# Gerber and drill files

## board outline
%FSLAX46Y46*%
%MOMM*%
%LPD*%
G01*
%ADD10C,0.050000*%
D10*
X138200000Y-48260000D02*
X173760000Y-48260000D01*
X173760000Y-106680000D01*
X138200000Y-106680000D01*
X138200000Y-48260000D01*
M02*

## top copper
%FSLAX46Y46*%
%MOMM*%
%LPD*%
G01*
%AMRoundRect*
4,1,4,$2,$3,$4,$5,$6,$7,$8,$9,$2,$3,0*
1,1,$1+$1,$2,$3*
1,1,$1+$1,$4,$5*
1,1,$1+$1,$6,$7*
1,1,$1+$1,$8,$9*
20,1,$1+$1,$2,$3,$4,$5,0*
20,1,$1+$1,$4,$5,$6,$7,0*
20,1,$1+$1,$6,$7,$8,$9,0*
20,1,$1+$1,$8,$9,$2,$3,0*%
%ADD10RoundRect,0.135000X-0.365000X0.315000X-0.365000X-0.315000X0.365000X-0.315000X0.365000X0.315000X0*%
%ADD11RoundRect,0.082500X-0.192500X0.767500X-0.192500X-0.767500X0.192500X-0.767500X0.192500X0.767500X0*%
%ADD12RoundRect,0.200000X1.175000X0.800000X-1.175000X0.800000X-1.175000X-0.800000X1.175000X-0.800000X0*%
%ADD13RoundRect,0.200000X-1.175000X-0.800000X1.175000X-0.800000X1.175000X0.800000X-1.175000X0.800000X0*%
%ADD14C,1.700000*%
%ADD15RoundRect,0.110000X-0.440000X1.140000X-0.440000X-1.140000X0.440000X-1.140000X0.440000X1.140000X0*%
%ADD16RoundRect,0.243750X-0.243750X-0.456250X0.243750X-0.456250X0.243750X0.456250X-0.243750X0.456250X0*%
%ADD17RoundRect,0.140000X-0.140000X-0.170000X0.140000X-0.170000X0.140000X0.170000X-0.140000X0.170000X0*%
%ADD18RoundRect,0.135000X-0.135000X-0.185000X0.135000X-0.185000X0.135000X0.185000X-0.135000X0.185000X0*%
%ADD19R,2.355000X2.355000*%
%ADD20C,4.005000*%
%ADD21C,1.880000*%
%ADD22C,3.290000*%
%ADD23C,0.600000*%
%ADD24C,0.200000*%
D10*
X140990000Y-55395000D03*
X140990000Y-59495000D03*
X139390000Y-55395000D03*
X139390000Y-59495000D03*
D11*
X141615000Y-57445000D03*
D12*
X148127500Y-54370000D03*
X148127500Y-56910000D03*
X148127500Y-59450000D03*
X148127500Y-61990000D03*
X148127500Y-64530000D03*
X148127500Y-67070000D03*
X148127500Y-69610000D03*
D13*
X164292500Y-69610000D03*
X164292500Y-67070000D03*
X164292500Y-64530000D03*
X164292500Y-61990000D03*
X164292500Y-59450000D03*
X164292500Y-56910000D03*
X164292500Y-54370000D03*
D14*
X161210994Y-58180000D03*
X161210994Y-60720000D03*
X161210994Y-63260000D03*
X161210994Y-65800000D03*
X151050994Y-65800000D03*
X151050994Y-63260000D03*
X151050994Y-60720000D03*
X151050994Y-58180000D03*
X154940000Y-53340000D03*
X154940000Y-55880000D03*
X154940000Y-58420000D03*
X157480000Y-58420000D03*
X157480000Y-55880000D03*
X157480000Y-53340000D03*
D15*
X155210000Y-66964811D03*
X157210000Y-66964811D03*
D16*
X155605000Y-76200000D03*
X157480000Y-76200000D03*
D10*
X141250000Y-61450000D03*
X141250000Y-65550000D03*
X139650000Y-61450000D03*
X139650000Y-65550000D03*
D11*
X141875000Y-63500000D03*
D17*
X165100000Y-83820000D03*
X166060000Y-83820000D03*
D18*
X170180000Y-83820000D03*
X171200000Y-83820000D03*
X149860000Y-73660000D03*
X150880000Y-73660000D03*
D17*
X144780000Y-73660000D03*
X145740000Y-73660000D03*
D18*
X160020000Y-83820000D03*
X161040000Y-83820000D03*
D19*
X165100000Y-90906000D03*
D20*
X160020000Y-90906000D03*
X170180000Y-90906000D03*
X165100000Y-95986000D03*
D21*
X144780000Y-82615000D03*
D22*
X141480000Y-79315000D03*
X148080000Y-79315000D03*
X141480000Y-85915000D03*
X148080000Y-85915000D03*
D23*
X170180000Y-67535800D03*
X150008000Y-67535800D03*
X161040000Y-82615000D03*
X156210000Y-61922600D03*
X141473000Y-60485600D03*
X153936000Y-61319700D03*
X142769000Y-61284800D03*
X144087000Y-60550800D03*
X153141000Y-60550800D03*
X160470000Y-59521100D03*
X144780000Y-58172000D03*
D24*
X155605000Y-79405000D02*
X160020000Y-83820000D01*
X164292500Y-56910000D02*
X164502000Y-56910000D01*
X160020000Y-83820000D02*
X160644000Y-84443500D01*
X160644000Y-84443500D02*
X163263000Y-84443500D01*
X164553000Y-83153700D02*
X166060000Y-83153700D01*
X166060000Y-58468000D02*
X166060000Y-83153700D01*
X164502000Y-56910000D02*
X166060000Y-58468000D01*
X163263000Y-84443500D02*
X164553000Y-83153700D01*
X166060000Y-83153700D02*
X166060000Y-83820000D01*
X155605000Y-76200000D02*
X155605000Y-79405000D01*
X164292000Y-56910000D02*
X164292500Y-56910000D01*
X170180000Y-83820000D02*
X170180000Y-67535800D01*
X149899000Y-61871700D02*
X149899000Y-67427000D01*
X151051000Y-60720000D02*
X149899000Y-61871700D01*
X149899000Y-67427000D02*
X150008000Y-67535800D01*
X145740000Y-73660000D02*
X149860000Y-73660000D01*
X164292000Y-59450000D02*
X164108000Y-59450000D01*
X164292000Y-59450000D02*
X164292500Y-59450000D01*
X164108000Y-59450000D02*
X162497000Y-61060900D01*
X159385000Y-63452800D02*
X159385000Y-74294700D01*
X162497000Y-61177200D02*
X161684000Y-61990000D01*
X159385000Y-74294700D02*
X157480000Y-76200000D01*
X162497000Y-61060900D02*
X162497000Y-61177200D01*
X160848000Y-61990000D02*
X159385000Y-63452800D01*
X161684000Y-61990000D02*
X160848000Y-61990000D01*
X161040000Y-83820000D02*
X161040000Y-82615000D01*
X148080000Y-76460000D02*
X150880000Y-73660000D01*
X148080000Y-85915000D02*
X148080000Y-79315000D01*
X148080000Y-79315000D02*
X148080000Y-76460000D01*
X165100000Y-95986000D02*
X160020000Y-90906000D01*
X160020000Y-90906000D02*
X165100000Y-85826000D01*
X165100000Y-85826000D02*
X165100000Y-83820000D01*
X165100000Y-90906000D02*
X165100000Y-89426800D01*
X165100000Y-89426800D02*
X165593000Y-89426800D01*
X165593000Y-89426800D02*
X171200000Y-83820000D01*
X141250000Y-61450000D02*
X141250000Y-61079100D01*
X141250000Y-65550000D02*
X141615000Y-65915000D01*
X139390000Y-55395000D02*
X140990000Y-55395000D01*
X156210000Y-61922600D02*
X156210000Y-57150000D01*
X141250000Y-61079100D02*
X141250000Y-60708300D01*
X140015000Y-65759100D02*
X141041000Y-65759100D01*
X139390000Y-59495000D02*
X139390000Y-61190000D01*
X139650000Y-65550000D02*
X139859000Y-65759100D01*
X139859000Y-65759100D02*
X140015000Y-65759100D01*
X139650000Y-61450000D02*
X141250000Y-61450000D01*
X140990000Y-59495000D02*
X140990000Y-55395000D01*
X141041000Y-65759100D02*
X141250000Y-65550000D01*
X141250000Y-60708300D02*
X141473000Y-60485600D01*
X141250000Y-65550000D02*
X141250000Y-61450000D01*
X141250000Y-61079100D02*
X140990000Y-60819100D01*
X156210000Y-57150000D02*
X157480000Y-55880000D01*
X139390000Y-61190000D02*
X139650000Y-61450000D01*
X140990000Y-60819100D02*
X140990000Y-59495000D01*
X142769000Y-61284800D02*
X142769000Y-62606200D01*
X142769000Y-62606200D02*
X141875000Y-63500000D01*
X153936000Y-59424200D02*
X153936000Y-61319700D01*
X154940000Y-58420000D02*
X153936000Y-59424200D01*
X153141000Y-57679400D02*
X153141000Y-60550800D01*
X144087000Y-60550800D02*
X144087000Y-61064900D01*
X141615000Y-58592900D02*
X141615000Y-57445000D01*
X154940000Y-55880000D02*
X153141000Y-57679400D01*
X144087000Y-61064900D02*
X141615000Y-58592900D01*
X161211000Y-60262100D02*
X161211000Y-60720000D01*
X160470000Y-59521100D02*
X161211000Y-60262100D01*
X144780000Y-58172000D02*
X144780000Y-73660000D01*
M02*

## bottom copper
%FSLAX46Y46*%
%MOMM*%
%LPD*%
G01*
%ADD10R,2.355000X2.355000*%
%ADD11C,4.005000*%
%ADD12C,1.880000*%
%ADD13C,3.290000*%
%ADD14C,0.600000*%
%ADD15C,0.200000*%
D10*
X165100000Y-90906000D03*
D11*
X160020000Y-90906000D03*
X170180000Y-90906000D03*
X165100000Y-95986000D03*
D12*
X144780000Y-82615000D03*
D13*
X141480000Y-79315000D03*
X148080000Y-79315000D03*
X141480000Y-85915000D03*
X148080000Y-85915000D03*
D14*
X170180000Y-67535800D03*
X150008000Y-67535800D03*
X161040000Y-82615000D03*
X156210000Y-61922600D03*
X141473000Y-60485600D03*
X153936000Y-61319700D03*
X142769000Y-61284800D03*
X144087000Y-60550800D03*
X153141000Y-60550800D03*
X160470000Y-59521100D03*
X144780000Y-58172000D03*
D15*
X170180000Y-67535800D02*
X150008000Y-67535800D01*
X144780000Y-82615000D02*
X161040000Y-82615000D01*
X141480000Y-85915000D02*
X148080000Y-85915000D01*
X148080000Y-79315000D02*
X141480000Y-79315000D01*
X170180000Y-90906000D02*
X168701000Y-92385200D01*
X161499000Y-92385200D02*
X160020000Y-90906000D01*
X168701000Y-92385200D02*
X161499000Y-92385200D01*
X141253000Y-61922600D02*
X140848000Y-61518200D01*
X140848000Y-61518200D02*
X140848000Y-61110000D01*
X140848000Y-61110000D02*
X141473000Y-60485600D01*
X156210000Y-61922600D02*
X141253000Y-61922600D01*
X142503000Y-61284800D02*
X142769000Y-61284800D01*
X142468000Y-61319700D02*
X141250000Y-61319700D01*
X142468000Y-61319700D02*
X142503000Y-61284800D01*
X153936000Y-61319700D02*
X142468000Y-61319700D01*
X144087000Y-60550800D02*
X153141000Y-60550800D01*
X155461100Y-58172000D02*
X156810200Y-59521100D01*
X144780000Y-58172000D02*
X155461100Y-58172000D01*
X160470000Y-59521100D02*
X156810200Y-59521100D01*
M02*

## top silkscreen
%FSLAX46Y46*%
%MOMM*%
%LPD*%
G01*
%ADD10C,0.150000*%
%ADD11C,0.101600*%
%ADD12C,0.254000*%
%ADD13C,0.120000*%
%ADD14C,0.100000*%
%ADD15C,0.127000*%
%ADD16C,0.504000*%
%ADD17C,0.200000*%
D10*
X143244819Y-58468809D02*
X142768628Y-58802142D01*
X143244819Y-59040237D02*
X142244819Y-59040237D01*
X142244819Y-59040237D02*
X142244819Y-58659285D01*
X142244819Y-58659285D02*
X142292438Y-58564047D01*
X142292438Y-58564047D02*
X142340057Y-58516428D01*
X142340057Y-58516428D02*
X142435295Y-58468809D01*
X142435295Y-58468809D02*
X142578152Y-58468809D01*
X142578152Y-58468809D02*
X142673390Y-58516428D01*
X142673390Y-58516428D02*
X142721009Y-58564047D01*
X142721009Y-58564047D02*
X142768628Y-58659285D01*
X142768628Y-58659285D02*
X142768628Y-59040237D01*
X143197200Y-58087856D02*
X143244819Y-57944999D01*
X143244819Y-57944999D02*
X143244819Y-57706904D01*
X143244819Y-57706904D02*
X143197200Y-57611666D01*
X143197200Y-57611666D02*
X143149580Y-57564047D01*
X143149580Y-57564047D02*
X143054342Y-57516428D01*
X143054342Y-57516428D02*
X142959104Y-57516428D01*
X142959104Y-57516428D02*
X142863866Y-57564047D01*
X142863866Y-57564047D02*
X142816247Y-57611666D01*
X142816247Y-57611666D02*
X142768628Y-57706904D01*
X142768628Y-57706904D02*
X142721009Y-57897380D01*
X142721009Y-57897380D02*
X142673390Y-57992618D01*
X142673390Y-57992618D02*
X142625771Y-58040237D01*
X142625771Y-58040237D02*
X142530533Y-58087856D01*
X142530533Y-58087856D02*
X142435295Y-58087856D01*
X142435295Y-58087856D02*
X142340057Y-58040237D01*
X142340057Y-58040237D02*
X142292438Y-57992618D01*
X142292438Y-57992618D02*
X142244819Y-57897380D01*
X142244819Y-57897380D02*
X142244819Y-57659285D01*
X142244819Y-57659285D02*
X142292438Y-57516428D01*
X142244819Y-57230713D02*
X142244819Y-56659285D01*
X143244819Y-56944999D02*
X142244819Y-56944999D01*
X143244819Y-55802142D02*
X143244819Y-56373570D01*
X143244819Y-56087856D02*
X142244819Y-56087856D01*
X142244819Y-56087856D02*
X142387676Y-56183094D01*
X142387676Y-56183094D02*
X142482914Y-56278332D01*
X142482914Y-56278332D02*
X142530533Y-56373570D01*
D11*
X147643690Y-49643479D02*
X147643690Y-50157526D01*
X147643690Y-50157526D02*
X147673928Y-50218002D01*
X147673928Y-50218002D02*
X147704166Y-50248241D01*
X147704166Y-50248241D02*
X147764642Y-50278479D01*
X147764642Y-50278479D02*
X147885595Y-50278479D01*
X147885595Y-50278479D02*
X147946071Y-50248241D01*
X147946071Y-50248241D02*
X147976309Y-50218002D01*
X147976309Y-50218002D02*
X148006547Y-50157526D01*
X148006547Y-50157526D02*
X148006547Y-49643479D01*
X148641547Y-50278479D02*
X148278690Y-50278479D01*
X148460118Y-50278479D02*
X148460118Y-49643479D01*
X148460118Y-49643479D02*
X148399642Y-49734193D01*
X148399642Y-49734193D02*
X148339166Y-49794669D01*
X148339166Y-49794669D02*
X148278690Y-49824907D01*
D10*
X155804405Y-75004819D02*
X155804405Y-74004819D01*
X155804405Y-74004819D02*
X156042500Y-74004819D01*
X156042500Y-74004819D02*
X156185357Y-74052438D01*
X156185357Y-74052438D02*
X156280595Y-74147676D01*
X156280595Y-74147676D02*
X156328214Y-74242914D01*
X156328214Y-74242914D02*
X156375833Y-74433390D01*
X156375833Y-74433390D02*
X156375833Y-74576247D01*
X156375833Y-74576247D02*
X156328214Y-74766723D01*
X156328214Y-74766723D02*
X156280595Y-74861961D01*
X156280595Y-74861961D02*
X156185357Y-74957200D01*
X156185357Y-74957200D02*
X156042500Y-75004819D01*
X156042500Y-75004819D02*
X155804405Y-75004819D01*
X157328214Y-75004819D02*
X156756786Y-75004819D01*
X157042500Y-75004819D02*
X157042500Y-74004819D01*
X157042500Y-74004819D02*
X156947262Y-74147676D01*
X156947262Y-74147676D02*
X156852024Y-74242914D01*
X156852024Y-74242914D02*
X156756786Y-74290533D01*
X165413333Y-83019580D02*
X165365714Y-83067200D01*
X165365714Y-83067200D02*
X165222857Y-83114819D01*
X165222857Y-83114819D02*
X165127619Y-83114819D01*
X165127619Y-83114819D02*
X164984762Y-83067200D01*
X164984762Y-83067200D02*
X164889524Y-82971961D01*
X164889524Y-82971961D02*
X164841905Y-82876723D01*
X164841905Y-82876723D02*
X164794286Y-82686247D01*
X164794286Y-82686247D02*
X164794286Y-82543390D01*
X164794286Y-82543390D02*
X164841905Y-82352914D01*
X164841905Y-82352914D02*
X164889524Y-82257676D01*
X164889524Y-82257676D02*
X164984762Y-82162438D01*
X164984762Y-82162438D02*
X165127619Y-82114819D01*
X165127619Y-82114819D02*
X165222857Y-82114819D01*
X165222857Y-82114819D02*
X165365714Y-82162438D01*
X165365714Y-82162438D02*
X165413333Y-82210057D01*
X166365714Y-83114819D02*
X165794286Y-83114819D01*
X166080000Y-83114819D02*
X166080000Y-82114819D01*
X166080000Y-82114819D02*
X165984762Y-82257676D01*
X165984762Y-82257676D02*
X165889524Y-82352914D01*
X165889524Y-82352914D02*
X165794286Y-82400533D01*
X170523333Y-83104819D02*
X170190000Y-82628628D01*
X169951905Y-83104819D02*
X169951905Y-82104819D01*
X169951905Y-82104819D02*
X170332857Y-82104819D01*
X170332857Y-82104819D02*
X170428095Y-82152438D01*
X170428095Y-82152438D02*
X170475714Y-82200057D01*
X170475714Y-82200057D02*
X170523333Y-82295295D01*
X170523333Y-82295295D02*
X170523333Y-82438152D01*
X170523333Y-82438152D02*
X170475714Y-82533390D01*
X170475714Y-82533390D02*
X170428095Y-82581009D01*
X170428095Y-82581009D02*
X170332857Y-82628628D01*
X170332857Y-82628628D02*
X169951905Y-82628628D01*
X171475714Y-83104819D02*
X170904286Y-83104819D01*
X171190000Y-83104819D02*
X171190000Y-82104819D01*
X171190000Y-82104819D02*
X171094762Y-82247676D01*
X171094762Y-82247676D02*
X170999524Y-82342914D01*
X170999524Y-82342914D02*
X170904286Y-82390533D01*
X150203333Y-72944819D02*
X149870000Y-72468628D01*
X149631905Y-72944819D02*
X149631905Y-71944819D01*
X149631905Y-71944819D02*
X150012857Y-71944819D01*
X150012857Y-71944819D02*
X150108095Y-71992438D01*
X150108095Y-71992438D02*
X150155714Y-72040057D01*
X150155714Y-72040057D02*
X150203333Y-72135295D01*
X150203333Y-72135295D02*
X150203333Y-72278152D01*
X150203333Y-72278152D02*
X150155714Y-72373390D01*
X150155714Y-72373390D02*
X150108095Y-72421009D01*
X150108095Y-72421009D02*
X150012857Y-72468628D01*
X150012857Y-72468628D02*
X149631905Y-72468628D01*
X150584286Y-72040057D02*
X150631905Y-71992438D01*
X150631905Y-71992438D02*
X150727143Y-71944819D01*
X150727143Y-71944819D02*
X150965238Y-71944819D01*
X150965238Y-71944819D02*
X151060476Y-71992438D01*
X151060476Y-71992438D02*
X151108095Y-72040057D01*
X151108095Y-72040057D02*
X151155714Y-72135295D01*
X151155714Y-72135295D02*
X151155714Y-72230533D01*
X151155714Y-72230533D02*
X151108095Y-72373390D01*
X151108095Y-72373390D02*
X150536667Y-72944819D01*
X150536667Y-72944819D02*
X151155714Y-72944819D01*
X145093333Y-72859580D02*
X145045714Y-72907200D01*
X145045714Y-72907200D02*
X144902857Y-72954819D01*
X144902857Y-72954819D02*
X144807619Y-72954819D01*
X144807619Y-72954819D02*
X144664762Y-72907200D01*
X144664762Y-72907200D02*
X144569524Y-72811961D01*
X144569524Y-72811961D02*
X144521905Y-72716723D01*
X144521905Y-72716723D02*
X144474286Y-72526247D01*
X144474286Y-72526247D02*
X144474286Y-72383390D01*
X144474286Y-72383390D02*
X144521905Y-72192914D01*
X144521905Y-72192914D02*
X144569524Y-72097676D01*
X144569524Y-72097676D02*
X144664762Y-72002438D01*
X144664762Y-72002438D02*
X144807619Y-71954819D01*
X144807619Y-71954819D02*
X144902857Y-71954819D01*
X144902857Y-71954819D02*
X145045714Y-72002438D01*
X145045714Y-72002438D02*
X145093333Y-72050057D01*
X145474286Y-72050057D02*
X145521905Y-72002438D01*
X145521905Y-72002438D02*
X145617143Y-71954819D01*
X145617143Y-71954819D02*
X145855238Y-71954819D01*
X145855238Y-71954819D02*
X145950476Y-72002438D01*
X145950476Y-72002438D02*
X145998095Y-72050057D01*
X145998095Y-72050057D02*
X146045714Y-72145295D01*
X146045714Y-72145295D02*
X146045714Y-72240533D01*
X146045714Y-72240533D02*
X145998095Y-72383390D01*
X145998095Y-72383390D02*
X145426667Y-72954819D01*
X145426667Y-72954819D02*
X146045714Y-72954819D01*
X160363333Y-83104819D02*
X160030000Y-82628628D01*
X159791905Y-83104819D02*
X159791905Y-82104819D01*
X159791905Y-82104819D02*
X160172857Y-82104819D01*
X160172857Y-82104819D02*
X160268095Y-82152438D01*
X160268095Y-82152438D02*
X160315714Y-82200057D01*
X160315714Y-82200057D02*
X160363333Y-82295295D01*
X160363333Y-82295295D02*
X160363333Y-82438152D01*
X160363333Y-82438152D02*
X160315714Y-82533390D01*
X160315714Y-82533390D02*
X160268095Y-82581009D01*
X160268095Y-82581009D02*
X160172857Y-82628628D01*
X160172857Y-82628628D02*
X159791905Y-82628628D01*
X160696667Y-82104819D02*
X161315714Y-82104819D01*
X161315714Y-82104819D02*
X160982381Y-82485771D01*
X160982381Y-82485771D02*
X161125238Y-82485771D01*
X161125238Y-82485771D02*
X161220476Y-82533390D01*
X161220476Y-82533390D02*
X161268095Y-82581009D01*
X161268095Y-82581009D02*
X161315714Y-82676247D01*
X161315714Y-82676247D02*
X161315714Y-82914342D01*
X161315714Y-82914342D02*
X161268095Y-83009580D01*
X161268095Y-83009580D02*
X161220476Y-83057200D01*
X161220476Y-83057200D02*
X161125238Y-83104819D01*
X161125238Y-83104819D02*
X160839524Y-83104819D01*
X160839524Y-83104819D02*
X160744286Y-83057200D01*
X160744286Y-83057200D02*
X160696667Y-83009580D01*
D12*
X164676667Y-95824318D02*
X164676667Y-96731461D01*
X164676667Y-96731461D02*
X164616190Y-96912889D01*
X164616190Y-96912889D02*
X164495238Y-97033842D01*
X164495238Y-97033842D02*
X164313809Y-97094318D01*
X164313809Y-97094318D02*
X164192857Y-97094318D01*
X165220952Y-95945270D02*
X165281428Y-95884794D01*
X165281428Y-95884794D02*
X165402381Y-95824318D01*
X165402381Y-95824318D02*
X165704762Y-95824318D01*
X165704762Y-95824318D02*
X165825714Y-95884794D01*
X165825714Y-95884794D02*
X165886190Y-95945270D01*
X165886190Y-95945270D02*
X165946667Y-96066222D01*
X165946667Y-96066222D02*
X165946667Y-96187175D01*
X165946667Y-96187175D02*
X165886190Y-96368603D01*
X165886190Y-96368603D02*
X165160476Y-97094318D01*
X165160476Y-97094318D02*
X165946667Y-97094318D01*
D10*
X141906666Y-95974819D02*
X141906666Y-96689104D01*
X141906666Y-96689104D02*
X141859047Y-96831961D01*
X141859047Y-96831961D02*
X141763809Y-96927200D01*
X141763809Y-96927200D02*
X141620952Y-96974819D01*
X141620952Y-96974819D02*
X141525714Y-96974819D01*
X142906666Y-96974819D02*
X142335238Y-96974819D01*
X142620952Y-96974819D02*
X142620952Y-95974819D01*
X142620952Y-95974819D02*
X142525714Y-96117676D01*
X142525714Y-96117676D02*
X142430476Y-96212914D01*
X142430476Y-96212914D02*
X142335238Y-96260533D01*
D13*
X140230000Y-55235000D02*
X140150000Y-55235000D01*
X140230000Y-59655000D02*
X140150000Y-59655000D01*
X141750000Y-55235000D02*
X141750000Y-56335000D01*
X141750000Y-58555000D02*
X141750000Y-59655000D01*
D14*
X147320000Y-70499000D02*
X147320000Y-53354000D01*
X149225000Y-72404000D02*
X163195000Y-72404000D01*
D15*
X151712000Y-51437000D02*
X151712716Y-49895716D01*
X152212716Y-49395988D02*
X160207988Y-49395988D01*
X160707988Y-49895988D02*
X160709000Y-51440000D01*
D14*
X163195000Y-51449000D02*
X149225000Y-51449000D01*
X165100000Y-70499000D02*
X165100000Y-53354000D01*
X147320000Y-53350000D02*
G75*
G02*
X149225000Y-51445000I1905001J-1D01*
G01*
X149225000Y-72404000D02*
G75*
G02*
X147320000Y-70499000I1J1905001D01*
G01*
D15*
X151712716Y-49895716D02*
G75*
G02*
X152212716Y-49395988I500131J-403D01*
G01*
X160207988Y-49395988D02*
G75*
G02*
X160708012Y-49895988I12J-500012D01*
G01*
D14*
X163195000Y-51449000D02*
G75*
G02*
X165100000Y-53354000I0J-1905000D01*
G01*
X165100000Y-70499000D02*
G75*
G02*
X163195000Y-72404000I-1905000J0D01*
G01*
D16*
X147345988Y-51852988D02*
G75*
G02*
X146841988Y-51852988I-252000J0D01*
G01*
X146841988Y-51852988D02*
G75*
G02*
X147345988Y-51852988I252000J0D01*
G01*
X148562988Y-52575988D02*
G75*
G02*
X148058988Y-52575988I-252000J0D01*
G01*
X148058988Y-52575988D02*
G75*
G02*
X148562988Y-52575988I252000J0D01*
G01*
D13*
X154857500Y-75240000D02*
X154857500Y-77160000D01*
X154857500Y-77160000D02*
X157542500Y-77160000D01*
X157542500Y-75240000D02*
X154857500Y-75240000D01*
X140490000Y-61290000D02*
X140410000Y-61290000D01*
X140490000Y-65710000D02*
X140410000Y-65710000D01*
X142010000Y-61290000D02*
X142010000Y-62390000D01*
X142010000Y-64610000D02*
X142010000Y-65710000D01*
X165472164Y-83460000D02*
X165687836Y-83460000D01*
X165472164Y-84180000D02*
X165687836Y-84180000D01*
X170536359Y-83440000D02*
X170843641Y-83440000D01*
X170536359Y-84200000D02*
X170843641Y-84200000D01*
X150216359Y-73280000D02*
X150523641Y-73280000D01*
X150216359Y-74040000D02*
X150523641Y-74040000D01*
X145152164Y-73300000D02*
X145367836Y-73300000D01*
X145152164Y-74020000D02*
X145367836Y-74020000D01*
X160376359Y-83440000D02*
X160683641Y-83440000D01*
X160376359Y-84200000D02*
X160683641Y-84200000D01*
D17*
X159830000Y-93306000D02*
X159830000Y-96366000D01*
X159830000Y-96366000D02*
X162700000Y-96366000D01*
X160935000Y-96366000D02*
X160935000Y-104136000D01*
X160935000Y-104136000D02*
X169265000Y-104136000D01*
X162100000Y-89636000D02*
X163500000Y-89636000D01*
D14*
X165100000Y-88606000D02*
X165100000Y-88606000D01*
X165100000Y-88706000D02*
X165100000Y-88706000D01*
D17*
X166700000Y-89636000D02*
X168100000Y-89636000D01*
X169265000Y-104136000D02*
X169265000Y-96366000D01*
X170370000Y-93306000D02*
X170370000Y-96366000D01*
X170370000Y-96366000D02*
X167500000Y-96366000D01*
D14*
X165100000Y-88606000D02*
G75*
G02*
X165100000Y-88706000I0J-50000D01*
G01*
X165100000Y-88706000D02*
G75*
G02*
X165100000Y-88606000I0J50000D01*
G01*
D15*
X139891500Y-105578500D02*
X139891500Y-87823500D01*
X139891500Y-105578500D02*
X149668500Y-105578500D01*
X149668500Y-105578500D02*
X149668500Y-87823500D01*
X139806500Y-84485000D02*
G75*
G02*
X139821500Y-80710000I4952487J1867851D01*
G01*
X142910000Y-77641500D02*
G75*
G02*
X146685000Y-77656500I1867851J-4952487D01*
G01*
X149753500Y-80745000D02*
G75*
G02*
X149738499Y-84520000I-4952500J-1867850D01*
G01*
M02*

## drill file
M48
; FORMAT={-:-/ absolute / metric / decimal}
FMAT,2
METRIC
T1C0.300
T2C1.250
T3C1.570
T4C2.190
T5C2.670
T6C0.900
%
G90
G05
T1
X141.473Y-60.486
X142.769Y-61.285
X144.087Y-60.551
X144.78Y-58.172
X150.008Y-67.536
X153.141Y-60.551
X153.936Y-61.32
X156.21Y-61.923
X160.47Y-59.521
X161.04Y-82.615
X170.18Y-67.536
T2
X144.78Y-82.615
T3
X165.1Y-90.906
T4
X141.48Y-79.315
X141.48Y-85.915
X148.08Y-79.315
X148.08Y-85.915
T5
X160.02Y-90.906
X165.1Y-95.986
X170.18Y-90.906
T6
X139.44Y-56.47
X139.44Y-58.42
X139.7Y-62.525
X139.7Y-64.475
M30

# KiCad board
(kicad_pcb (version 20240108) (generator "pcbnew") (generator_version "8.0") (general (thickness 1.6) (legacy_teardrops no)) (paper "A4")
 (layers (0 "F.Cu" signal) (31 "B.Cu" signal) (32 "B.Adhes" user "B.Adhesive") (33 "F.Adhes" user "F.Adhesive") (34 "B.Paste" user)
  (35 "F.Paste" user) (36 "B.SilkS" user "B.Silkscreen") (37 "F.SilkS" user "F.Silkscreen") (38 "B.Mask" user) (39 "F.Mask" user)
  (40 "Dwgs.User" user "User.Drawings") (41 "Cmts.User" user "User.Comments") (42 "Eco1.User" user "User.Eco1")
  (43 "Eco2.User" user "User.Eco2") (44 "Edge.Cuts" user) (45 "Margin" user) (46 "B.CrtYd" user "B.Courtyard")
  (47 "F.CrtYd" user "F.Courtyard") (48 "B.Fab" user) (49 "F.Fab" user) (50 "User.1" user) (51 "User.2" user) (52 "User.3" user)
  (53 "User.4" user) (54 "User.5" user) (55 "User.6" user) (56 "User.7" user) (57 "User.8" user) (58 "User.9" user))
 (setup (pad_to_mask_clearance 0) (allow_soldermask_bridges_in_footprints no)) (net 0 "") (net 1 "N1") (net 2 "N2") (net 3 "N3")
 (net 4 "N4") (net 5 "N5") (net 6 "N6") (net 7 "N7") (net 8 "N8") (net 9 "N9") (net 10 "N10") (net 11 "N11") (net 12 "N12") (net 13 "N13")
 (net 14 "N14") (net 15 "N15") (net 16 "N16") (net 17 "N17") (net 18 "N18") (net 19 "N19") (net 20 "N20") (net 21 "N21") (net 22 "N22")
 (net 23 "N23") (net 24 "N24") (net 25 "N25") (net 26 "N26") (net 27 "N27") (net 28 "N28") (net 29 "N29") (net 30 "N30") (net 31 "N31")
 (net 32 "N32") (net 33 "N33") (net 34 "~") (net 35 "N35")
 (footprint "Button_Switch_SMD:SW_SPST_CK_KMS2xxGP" (layer "F.Cu") (at 140.19 57.445 -90)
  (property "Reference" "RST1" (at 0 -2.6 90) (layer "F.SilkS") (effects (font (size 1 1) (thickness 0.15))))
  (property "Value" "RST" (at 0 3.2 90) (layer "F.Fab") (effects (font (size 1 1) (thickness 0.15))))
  (fp_line (start -2.21 -0.04) (end -2.21 0.04) (stroke (width 0.12) (type default)) (layer "F.SilkS"))
  (fp_line (start 2.21 -0.04) (end 2.21 0.04) (stroke (width 0.12) (type default)) (layer "F.SilkS"))
  (fp_line (start -2.21 -1.56) (end -1.11 -1.56) (stroke (width 0.12) (type solid)) (layer "F.SilkS"))
  (fp_line (start 1.11 -1.56) (end 2.21 -1.56) (stroke (width 0.12) (type solid)) (layer "F.SilkS"))
  (pad "" np_thru_hole circle (at -0.975 0.75 270) (size 0.9 0.9) (drill 0.9) (layers "F&B.Cu" "*.Mask"))
  (pad "" np_thru_hole circle (at 0.975 0.75 270) (size 0.9 0.9) (drill 0.9) (layers "F&B.Cu" "*.Mask"))
  (pad "1" smd roundrect (at -2.05 -0.8 270) (size 0.9 1) (layers "F.Cu" "F.Paste" "F.Mask") (roundrect_rratio 0.15) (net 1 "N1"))
  (pad "1" smd roundrect (at 2.05 -0.8 270) (size 0.9 1) (layers "F.Cu" "F.Paste" "F.Mask") (roundrect_rratio 0.15) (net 1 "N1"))
  (pad "2" smd roundrect (at -2.05 0.8 270) (size 0.9 1) (layers "F.Cu" "F.Paste" "F.Mask") (roundrect_rratio 0.15) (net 1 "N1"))
  (pad "2" smd roundrect (at 2.05 0.8 270) (size 0.9 1) (layers "F.Cu" "F.Paste" "F.Mask") (roundrect_rratio 0.15) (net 1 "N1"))
  (pad "SH" smd roundrect (at 0 -1.425 270) (size 1.7 0.55) (layers "F.Cu" "F.Paste" "F.Mask") (roundrect_rratio 0.15) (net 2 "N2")))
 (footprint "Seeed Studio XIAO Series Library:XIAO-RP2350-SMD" (layer "F.Cu") (at 156.1275 61.99)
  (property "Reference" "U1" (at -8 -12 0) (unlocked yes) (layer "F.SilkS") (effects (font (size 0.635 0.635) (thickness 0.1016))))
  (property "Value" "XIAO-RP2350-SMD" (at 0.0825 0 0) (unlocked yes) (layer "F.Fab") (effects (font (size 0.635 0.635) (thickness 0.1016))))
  (fp_line (start -8.8075 8.509) (end -8.8075 -8.636) (stroke (width 0.1) (type solid)) (layer "F.SilkS"))
  (fp_line (start -6.9025 10.414) (end 7.0675 10.414) (stroke (width 0.1) (type solid)) (layer "F.SilkS"))
  (fp_line (start -4.4155 -10.553) (end -4.414784 -12.094284) (stroke (width 0.127) (type solid)) (layer "F.SilkS"))
  (fp_line (start -3.914784 -12.594012) (end 4.080488 -12.594012) (stroke (width 0.127) (type solid)) (layer "F.SilkS"))
  (fp_line (start 4.580488 -12.094012) (end 4.5815 -10.55) (stroke (width 0.127) (type solid)) (layer "F.SilkS"))
  (fp_line (start 7.0675 -10.541) (end -6.9025 -10.541) (stroke (width 0.1) (type solid)) (layer "F.SilkS"))
  (fp_line (start 8.9725 8.509) (end 8.9725 -8.636) (stroke (width 0.1) (type solid)) (layer "F.SilkS"))
  (fp_arc (start -8.8075 -8.64) (mid -8.249538 -9.987038) (end -6.9025 -10.545) (stroke (width 0.1) (type solid)) (layer "F.SilkS"))
  (fp_arc (start -6.9025 10.414) (mid -8.249538 9.856038) (end -8.8075 8.509) (stroke (width 0.1) (type solid)) (layer "F.SilkS"))
  (fp_arc (start -4.414784 -12.094284) (mid -4.268203 -12.447623) (end -3.914784 -12.594012) (stroke (width 0.127) (type default))
   (layer "F.SilkS"))
  (fp_arc (start 4.080488 -12.594012) (mid 4.434053 -12.44757) (end 4.580488 -12.094012) (stroke (width 0.127) (type default))
   (layer "F.SilkS"))
  (fp_arc (start 7.0675 -10.541) (mid 8.414538 -9.983038) (end 8.9725 -8.636) (stroke (width 0.1) (type solid)) (layer "F.SilkS"))
  (fp_arc (start 8.9725 8.509) (mid 8.414538 9.856038) (end 7.0675 10.414) (stroke (width 0.1) (type solid)) (layer "F.SilkS"))
  (fp_circle (center -9.033512 -10.137012) (end -9.033512 -10.391012) (stroke (width 0.5) (type solid)) (fill solid) (layer "F.SilkS"))
  (fp_circle (center -7.816512 -9.414012) (end -7.816512 -9.668012) (stroke (width 0.5) (type solid)) (fill solid) (layer "F.SilkS"))
  (pad "1" smd roundrect (at -8 -7.62 180) (size 2.75 2) (layers "F.Cu" "F.Paste" "F.Mask") (roundrect_rratio 0.1) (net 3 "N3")
   (thermal_bridge_angle 45))
  (pad "2" smd roundrect (at -8 -5.08 180) (size 2.75 2) (layers "F.Cu" "F.Paste" "F.Mask") (roundrect_rratio 0.1) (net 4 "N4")
   (thermal_bridge_angle 45))
  (pad "3" smd roundrect (at -8 -2.54 180) (size 2.75 2) (layers "F.Cu" "F.Paste" "F.Mask") (roundrect_rratio 0.1) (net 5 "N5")
   (thermal_bridge_angle 45))
  (pad "4" smd roundrect (at -8 0 180) (size 2.75 2) (layers "F.Cu" "F.Paste" "F.Mask") (roundrect_rratio 0.1) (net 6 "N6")
   (thermal_bridge_angle 45))
  (pad "5" smd roundrect (at -8 2.54 180) (size 2.75 2) (layers "F.Cu" "F.Paste" "F.Mask") (roundrect_rratio 0.1) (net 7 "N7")
   (thermal_bridge_angle 45))
  (pad "6" smd roundrect (at -8 5.08 180) (size 2.75 2) (layers "F.Cu" "F.Paste" "F.Mask") (roundrect_rratio 0.1) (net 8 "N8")
   (thermal_bridge_angle 45))
  (pad "7" smd roundrect (at -8 7.62 180) (size 2.75 2) (layers "F.Cu" "F.Paste" "F.Mask") (roundrect_rratio 0.1) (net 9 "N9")
   (thermal_bridge_angle 45))
  (pad "8" smd roundrect (at 8.165 7.62) (size 2.75 2) (layers "F.Cu" "F.Paste" "F.Mask") (roundrect_rratio 0.1) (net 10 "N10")
   (thermal_bridge_angle 45))
  (pad "9" smd roundrect (at 8.165 5.08) (size 2.75 2) (layers "F.Cu" "F.Paste" "F.Mask") (roundrect_rratio 0.1) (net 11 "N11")
   (thermal_bridge_angle 45))
  (pad "10" smd roundrect (at 8.165 2.54) (size 2.75 2) (layers "F.Cu" "F.Paste" "F.Mask") (roundrect_rratio 0.1) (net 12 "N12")
   (thermal_bridge_angle 45))
  (pad "11" smd roundrect (at 8.165 0) (size 2.75 2) (layers "F.Cu" "F.Paste" "F.Mask") (roundrect_rratio 0.1) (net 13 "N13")
   (thermal_bridge_angle 45))
  (pad "12" smd roundrect (at 8.165 -2.54) (size 2.75 2) (layers "F.Cu" "F.Paste" "F.Mask") (roundrect_rratio 0.1) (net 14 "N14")
   (thermal_bridge_angle 45))
  (pad "13" smd roundrect (at 8.165 -5.08) (size 2.75 2) (layers "F.Cu" "F.Paste" "F.Mask") (roundrect_rratio 0.1) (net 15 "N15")
   (thermal_bridge_angle 45))
  (pad "14" smd roundrect (at 8.165 -7.62) (size 2.75 2) (layers "F.Cu" "F.Paste" "F.Mask") (roundrect_rratio 0.1) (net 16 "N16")
   (thermal_bridge_angle 45))
  (pad "15" smd circle (at 5.083494 -3.81 180) (size 1.7 1.7) (layers "F.Cu" "F.Paste" "F.Mask") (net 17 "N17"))
  (pad "16" smd circle (at 5.083494 -1.27 180) (size 1.7 1.7) (layers "F.Cu" "F.Paste" "F.Mask") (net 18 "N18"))
  (pad "17" smd circle (at 5.083494 1.27 180) (size 1.7 1.7) (layers "F.Cu" "F.Paste" "F.Mask") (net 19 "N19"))
  (pad "18" smd circle (at 5.083494 3.81 180) (size 1.7 1.7) (layers "F.Cu" "F.Paste" "F.Mask") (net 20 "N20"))
  (pad "19" smd circle (at -5.076506 3.81 180) (size 1.7 1.7) (layers "F.Cu" "F.Paste" "F.Mask") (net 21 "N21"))
  (pad "20" smd circle (at -5.076506 1.27 180) (size 1.7 1.7) (layers "F.Cu" "F.Paste" "F.Mask") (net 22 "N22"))
  (pad "21" smd circle (at -5.076506 -1.27 180) (size 1.7 1.7) (layers "F.Cu" "F.Paste" "F.Mask") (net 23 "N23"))
  (pad "22" smd circle (at -5.076506 -3.81 180) (size 1.7 1.7) (layers "F.Cu" "F.Paste" "F.Mask") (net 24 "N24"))
  (pad "23" smd circle (at -1.1875 -8.65 180) (size 1.7 1.7) (layers "F.Cu" "F.Paste" "F.Mask") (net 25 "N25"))
  (pad "24" smd circle (at -1.1875 -6.11 180) (size 1.7 1.7) (layers "F.Cu" "F.Paste" "F.Mask") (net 2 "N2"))
  (pad "25" smd circle (at -1.1875 -3.57 180) (size 1.7 1.7) (layers "F.Cu" "F.Paste" "F.Mask") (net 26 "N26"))
  (pad "26" smd circle (at 1.3525 -3.57 180) (size 1.7 1.7) (layers "F.Cu" "F.Paste" "F.Mask") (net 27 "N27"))
  (pad "27" smd circle (at 1.3525 -6.11 180) (size 1.7 1.7) (layers "F.Cu" "F.Paste" "F.Mask") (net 1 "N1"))
  (pad "28" smd circle (at 1.3525 -8.65 180) (size 1.7 1.7) (layers "F.Cu" "F.Paste" "F.Mask") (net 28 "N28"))
  (pad "29" smd roundrect (at -0.9175 4.974811 270) (size 2.5 1.1) (layers "F.Cu" "F.Paste" "F.Mask") (roundrect_rratio 0.1) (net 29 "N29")
   (thermal_bridge_angle 45))
  (pad "30" smd roundrect (at 1.0825 4.974811 270) (size 2.5 1.1) (layers "F.Cu" "F.Paste" "F.Mask") (roundrect_rratio 0.1) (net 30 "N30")
   (thermal_bridge_angle 45)))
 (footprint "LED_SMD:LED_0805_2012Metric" (layer "F.Cu") (at 156.5425 76.2)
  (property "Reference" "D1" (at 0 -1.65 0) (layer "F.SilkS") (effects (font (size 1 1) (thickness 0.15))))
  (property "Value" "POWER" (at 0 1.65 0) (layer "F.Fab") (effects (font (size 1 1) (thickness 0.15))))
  (fp_line (start -1.685 -0.96) (end -1.685 0.96) (stroke (width 0.12) (type solid)) (layer "F.SilkS"))
  (fp_line (start -1.685 0.96) (end 1 0.96) (stroke (width 0.12) (type solid)) (layer "F.SilkS"))
  (fp_line (start 1 -0.96) (end -1.685 -0.96) (stroke (width 0.12) (type solid)) (layer "F.SilkS"))
  (pad "1" smd roundrect (at -0.9375 0) (size 0.975 1.4) (layers "F.Cu" "F.Paste" "F.Mask") (roundrect_rratio 0.25) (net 15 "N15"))
  (pad "2" smd roundrect (at 0.9375 0) (size 0.975 1.4) (layers "F.Cu" "F.Paste" "F.Mask") (roundrect_rratio 0.25) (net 14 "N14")))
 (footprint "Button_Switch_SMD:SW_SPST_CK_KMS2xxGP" (layer "F.Cu") (at 140.45 63.5 -90)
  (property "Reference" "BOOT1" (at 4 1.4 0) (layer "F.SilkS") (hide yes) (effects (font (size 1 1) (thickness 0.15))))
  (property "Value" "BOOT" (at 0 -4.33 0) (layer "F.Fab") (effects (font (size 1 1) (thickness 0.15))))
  (fp_line (start -2.21 -0.04) (end -2.21 0.04) (stroke (width 0.12) (type default)) (layer "F.SilkS"))
  (fp_line (start 2.21 -0.04) (end 2.21 0.04) (stroke (width 0.12) (type default)) (layer "F.SilkS"))
  (fp_line (start -2.21 -1.56) (end -1.11 -1.56) (stroke (width 0.12) (type solid)) (layer "F.SilkS"))
  (fp_line (start 1.11 -1.56) (end 2.21 -1.56) (stroke (width 0.12) (type solid)) (layer "F.SilkS"))
  (pad "" np_thru_hole circle (at -0.975 0.75 270) (size 0.9 0.9) (drill 0.9) (layers "F&B.Cu" "*.Mask"))
  (pad "" np_thru_hole circle (at 0.975 0.75 270) (size 0.9 0.9) (drill 0.9) (layers "F&B.Cu" "*.Mask"))
  (pad "1" smd roundrect (at -2.05 -0.8 270) (size 0.9 1) (layers "F.Cu" "F.Paste" "F.Mask") (roundrect_rratio 0.15) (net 1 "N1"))
  (pad "1" smd roundrect (at 2.05 -0.8 270) (size 0.9 1) (layers "F.Cu" "F.Paste" "F.Mask") (roundrect_rratio 0.15) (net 1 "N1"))
  (pad "2" smd roundrect (at -2.05 0.8 270) (size 0.9 1) (layers "F.Cu" "F.Paste" "F.Mask") (roundrect_rratio 0.15) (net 1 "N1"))
  (pad "2" smd roundrect (at 2.05 0.8 270) (size 0.9 1) (layers "F.Cu" "F.Paste" "F.Mask") (roundrect_rratio 0.15) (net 1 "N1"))
  (pad "SH" smd roundrect (at 0 -1.425 270) (size 1.7 0.55) (layers "F.Cu" "F.Paste" "F.Mask") (roundrect_rratio 0.15) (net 26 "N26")))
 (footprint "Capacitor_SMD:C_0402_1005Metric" (layer "F.Cu") (at 165.58 83.82)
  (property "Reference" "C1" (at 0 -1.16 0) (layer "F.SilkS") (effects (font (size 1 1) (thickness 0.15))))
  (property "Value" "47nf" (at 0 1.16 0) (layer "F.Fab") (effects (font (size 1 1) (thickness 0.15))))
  (fp_line (start -0.107836 -0.36) (end 0.107836 -0.36) (stroke (width 0.12) (type solid)) (layer "F.SilkS"))
  (fp_line (start -0.107836 0.36) (end 0.107836 0.36) (stroke (width 0.12) (type solid)) (layer "F.SilkS"))
  (pad "1" smd roundrect (at -0.48 0) (size 0.56 0.62) (layers "F.Cu" "F.Paste" "F.Mask") (roundrect_rratio 0.25) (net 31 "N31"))
  (pad "2" smd roundrect (at 0.48 0) (size 0.56 0.62) (layers "F.Cu" "F.Paste" "F.Mask") (roundrect_rratio 0.25) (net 15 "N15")))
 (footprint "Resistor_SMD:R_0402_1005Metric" (layer "F.Cu") (at 170.69 83.82)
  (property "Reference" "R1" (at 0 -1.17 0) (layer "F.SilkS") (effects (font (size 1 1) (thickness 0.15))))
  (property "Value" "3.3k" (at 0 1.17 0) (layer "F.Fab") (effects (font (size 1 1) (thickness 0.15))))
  (fp_line (start -0.153641 -0.38) (end 0.153641 -0.38) (stroke (width 0.12) (type solid)) (layer "F.SilkS"))
  (fp_line (start -0.153641 0.38) (end 0.153641 0.38) (stroke (width 0.12) (type solid)) (layer "F.SilkS"))
  (pad "1" smd roundrect (at -0.51 0) (size 0.54 0.64) (layers "F.Cu" "F.Paste" "F.Mask") (roundrect_rratio 0.25) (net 23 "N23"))
  (pad "2" smd roundrect (at 0.51 0) (size 0.54 0.64) (layers "F.Cu" "F.Paste" "F.Mask") (roundrect_rratio 0.25) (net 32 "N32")))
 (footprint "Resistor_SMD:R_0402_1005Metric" (layer "F.Cu") (at 150.37 73.66)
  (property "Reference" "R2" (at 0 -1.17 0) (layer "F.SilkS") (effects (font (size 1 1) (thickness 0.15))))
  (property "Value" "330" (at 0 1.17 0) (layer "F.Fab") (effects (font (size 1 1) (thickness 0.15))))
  (fp_line (start -0.153641 -0.38) (end 0.153641 -0.38) (stroke (width 0.12) (type solid)) (layer "F.SilkS"))
  (fp_line (start -0.153641 0.38) (end 0.153641 0.38) (stroke (width 0.12) (type solid)) (layer "F.SilkS"))
  (pad "1" smd roundrect (at -0.51 0) (size 0.54 0.64) (layers "F.Cu" "F.Paste" "F.Mask") (roundrect_rratio 0.25) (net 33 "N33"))
  (pad "2" smd roundrect (at 0.51 0) (size 0.54 0.64) (layers "F.Cu" "F.Paste" "F.Mask") (roundrect_rratio 0.25) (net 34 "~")))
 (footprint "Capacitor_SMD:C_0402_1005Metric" (layer "F.Cu") (at 145.26 73.66)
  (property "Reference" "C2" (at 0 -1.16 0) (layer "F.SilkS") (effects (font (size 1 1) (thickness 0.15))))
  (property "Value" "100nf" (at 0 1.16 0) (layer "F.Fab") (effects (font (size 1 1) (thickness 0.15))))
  (fp_line (start -0.107836 -0.36) (end 0.107836 -0.36) (stroke (width 0.12) (type solid)) (layer "F.SilkS"))
  (fp_line (start -0.107836 0.36) (end 0.107836 0.36) (stroke (width 0.12) (type solid)) (layer "F.SilkS"))
  (pad "1" smd roundrect (at -0.48 0) (size 0.56 0.62) (layers "F.Cu" "F.Paste" "F.Mask") (roundrect_rratio 0.25) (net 18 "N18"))
  (pad "2" smd roundrect (at 0.48 0) (size 0.56 0.62) (layers "F.Cu" "F.Paste" "F.Mask") (roundrect_rratio 0.25) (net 33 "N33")))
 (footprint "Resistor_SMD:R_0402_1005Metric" (layer "F.Cu") (at 160.53 83.82)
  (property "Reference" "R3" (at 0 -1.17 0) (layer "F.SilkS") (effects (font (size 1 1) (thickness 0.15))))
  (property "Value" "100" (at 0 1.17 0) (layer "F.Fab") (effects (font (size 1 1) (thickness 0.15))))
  (fp_line (start -0.153641 -0.38) (end 0.153641 -0.38) (stroke (width 0.12) (type solid)) (layer "F.SilkS"))
  (fp_line (start -0.153641 0.38) (end 0.153641 0.38) (stroke (width 0.12) (type solid)) (layer "F.SilkS"))
  (pad "1" smd roundrect (at -0.51 0) (size 0.54 0.64) (layers "F.Cu" "F.Paste" "F.Mask") (roundrect_rratio 0.25) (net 15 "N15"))
  (pad "2" smd roundrect (at 0.51 0) (size 0.54 0.64) (layers "F.Cu" "F.Paste" "F.Mask") (roundrect_rratio 0.25) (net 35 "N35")))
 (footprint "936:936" (layer "F.Cu") (at 165.1 90.906)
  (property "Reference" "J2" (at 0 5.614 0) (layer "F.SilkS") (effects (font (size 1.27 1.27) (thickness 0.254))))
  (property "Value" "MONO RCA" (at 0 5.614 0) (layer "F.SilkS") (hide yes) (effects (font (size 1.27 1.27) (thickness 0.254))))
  (fp_line (start -5.27 2.4) (end -5.27 5.46) (stroke (width 0.2) (type solid)) (layer "F.SilkS"))
  (fp_line (start -5.27 5.46) (end -2.4 5.46) (stroke (width 0.2) (type solid)) (layer "F.SilkS"))
  (fp_line (start -4.165 5.46) (end -4.165 13.23) (stroke (width 0.2) (type solid)) (layer "F.SilkS"))
  (fp_line (start -4.165 13.23) (end 4.165 13.23) (stroke (width 0.2) (type solid)) (layer "F.SilkS"))
  (fp_line (start -3 -1.27) (end -1.6 -1.27) (stroke (width 0.2) (type solid)) (layer "F.SilkS"))
  (fp_line (start 0 -2.3) (end 0 -2.3) (stroke (width 0.1) (type solid)) (layer "F.SilkS"))
  (fp_line (start 0 -2.2) (end 0 -2.2) (stroke (width 0.1) (type solid)) (layer "F.SilkS"))
  (fp_line (start 1.6 -1.27) (end 3 -1.27) (stroke (width 0.2) (type solid)) (layer "F.SilkS"))
  (fp_line (start 4.165 13.23) (end 4.165 5.46) (stroke (width 0.2) (type solid)) (layer "F.SilkS"))
  (fp_line (start 5.27 2.4) (end 5.27 5.46) (stroke (width 0.2) (type solid)) (layer "F.SilkS"))
  (fp_line (start 5.27 5.46) (end 2.4 5.46) (stroke (width 0.2) (type solid)) (layer "F.SilkS"))
  (fp_arc (start 0 -2.3) (mid 0.05 -2.25) (end 0 -2.2) (stroke (width 0.1) (type solid)) (layer "F.SilkS"))
  (fp_arc (start 0 -2.2) (mid -0.05 -2.25) (end 0 -2.3) (stroke (width 0.1) (type solid)) (layer "F.SilkS"))
  (pad "1" thru_hole rect (at 0 0) (size 2.355 2.355) (drill 1.57) (layers "*.Cu" "*.Mask") (remove_unused_layers no) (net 32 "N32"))
  (pad "MH1" thru_hole circle (at -5.08 0) (size 4.005 4.005) (drill 2.67) (layers "*.Cu" "*.Mask") (remove_unused_layers no) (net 31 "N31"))
  (pad "MH2" thru_hole circle (at 5.08 0) (size 4.005 4.005) (drill 2.67) (layers "*.Cu" "*.Mask") (remove_unused_layers no) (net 31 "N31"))
  (pad "MH3" thru_hole circle (at 0 5.08) (size 4.005 4.005) (drill 2.67) (layers "*.Cu" "*.Mask") (remove_unused_layers no) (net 31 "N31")))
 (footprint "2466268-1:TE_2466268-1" (layer "F.Cu") (at 144.78 82.615)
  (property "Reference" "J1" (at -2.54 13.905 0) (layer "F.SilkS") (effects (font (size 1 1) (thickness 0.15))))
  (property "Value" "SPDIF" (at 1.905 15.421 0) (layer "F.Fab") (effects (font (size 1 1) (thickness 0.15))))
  (fp_line (start -4.8885 22.9635) (end -4.8885 5.2085) (stroke (width 0.127) (type solid)) (layer "F.SilkS"))
  (fp_line (start -4.8885 22.9635) (end 4.8885 22.9635) (stroke (width 0.127) (type solid)) (layer "F.SilkS"))
  (fp_line (start 4.8885 22.9635) (end 4.8885 5.2085) (stroke (width 0.127) (type solid)) (layer "F.SilkS"))
  (fp_arc (start -4.9735 1.87) (mid -5.313985 -0.018883) (end -4.9585 -1.905) (stroke (width 0.127) (type solid)) (layer "F.SilkS"))
  (fp_arc (start -1.87 -4.9735) (mid 0.018883 -5.313985) (end 1.905 -4.9585) (stroke (width 0.127) (type solid)) (layer "F.SilkS"))
  (fp_arc (start 4.9735 -1.87) (mid 5.313984 0.018883) (end 4.9585 1.905) (stroke (width 0.127) (type solid)) (layer "F.SilkS"))
  (pad "1" thru_hole circle (at 0 0) (size 1.88 1.88) (drill 1.25) (layers "*.Cu" "*.Mask") (remove_unused_layers no) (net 35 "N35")
   (solder_mask_margin 0.102))
  (pad "2" thru_hole circle (at -3.3 -3.3) (size 3.29 3.29) (drill 2.19) (layers "*.Cu" "*.Mask") (remove_unused_layers no) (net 34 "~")
   (solder_mask_margin 0.102))
  (pad "3" thru_hole circle (at 3.3 -3.3) (size 3.29 3.29) (drill 2.19) (layers "*.Cu" "*.Mask") (remove_unused_layers no) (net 34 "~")
   (solder_mask_margin 0.102))
  (pad "4" thru_hole circle (at -3.3 3.3) (size 3.29 3.29) (drill 2.19) (layers "*.Cu" "*.Mask") (remove_unused_layers no) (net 34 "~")
   (solder_mask_margin 0.102))
  (pad "5" thru_hole circle (at 3.3 3.3) (size 3.29 3.29) (drill 2.19) (layers "*.Cu" "*.Mask") (remove_unused_layers no) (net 34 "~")
   (solder_mask_margin 0.102)))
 (gr_rect (start 138.2 48.26) (end 173.76 106.68) (stroke (width 0.05) (type default)) (fill none) (layer "Edge.Cuts"))
 (segment (start 155.605 79.405) (end 160.02 83.82) (width 0.2) (layer "F.Cu") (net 15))
 (segment (start 164.2925 56.91) (end 164.502 56.91) (width 0.2) (layer "F.Cu") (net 15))
 (segment (start 160.02 83.82) (end 160.644 84.4435) (width 0.2) (layer "F.Cu") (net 15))
 (segment (start 160.644 84.4435) (end 163.263 84.4435) (width 0.2) (layer "F.Cu") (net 15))
 (segment (start 164.553 83.1537) (end 166.06 83.1537) (width 0.2) (layer "F.Cu") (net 15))
 (segment (start 166.06 58.468) (end 166.06 83.1537) (width 0.2) (layer "F.Cu") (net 15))
 (segment (start 164.502 56.91) (end 166.06 58.468) (width 0.2) (layer "F.Cu") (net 15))
 (segment (start 163.263 84.4435) (end 164.553 83.1537) (width 0.2) (layer "F.Cu") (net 15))
 (segment (start 166.06 83.1537) (end 166.06 83.82) (width 0.2) (layer "F.Cu") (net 15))
 (segment (start 155.605 76.2) (end 155.605 79.405) (width 0.2) (layer "F.Cu") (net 15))
 (segment (start 164.292 56.91) (end 164.2925 56.91) (width 0.2) (layer "F.Cu") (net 15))
 (segment (start 170.18 83.82) (end 170.18 67.5358) (width 0.2) (layer "F.Cu") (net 23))
 (segment (start 149.899 61.8717) (end 149.899 67.427) (width 0.2) (layer "F.Cu") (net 23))
 (segment (start 151.051 60.72) (end 149.899 61.8717) (width 0.2) (layer "F.Cu") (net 23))
 (segment (start 149.899 67.427) (end 150.008 67.5358) (width 0.2) (layer "F.Cu") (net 23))
 (via (at 170.18 67.5358) (size 0.6) (drill 0.3) (layers "F.Cu" "B.Cu") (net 23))
 (via (at 150.008 67.5358) (size 0.6) (drill 0.3) (layers "F.Cu" "B.Cu") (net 23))
 (segment (start 170.18 67.5358) (end 150.008 67.5358) (width 0.2) (layer "B.Cu") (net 23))
 (segment (start 145.74 73.66) (end 149.86 73.66) (width 0.2) (layer "F.Cu") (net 33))
 (segment (start 164.292 59.45) (end 164.108 59.45) (width 0.2) (layer "F.Cu") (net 14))
 (segment (start 164.292 59.45) (end 164.2925 59.45) (width 0.2) (layer "F.Cu") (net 14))
 (segment (start 164.108 59.45) (end 162.497 61.0609) (width 0.2) (layer "F.Cu") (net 14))
 (segment (start 159.385 63.4528) (end 159.385 74.2947) (width 0.2) (layer "F.Cu") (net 14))
 (segment (start 162.497 61.1772) (end 161.684 61.99) (width 0.2) (layer "F.Cu") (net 14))
 (segment (start 159.385 74.2947) (end 157.48 76.2) (width 0.2) (layer "F.Cu") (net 14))
 (segment (start 162.497 61.0609) (end 162.497 61.1772) (width 0.2) (layer "F.Cu") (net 14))
 (segment (start 160.848 61.99) (end 159.385 63.4528) (width 0.2) (layer "F.Cu") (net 14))
 (segment (start 161.684 61.99) (end 160.848 61.99) (width 0.2) (layer "F.Cu") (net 14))
 (segment (start 161.04 83.82) (end 161.04 82.615) (width 0.2) (layer "F.Cu") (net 35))
 (via (at 161.04 82.615) (size 0.6) (drill 0.3) (layers "F.Cu" "B.Cu") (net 35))
 (segment (start 144.78 82.615) (end 161.04 82.615) (width 0.2) (layer "B.Cu") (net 35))
 (segment (start 148.08 76.46) (end 150.88 73.66) (width 0.2) (layer "F.Cu") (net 34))
 (segment (start 148.08 85.915) (end 148.08 79.315) (width 0.2) (layer "F.Cu") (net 34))
 (segment (start 148.08 79.315) (end 148.08 76.46) (width 0.2) (layer "F.Cu") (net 34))
 (segment (start 141.48 85.915) (end 148.08 85.915) (width 0.2) (layer "B.Cu") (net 34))
 (segment (start 148.08 79.315) (end 141.48 79.315) (width 0.2) (layer "B.Cu") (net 34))
 (segment (start 165.1 95.986) (end 160.02 90.906) (width 0.2) (layer "F.Cu") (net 31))
 (segment (start 160.02 90.906) (end 165.1 85.826) (width 0.2) (layer "F.Cu") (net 31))
 (segment (start 165.1 85.826) (end 165.1 83.82) (width 0.2) (layer "F.Cu") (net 31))
 (segment (start 170.18 90.906) (end 168.701 92.3852) (width 0.2) (layer "B.Cu") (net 31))
 (segment (start 161.499 92.3852) (end 160.02 90.906) (width 0.2) (layer "B.Cu") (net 31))
 (segment (start 168.701 92.3852) (end 161.499 92.3852) (width 0.2) (layer "B.Cu") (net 31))
 (segment (start 165.1 90.906) (end 165.1 89.4268) (width 0.2) (layer "F.Cu") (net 32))
 (segment (start 165.1 89.4268) (end 165.593 89.4268) (width 0.2) (layer "F.Cu") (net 32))
 (segment (start 165.593 89.4268) (end 171.2 83.82) (width 0.2) (layer "F.Cu") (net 32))
 (segment (start 141.25 61.45) (end 141.25 61.0791) (width 0.2) (layer "F.Cu") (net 1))
 (segment (start 141.25 65.55) (end 141.615 65.915) (width 0.2) (layer "F.Cu") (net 1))
 (segment (start 139.39 55.395) (end 140.99 55.395) (width 0.2) (layer "F.Cu") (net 1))
 (segment (start 156.21 61.9226) (end 156.21 57.15) (width 0.2) (layer "F.Cu") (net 1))
 (segment (start 141.25 61.0791) (end 141.25 60.7083) (width 0.2) (layer "F.Cu") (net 1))
 (segment (start 140.015 65.7591) (end 141.041 65.7591) (width 0.2) (layer "F.Cu") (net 1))
 (segment (start 139.39 59.495) (end 139.39 61.19) (width 0.2) (layer "F.Cu") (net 1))
 (segment (start 139.65 65.55) (end 139.859 65.7591) (width 0.2) (layer "F.Cu") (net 1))
 (segment (start 139.859 65.7591) (end 140.015 65.7591) (width 0.2) (layer "F.Cu") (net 1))
 (segment (start 139.65 61.45) (end 141.25 61.45) (width 0.2) (layer "F.Cu") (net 1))
 (segment (start 140.99 59.495) (end 140.99 55.395) (width 0.2) (layer "F.Cu") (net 1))
 (segment (start 141.041 65.7591) (end 141.25 65.55) (width 0.2) (layer "F.Cu") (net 1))
 (segment (start 141.25 60.7083) (end 141.473 60.4856) (width 0.2) (layer "F.Cu") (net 1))
 (segment (start 141.25 65.55) (end 141.25 61.45) (width 0.2) (layer "F.Cu") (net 1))
 (segment (start 141.25 61.0791) (end 140.99 60.8191) (width 0.2) (layer "F.Cu") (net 1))
 (segment (start 156.21 57.15) (end 157.48 55.88) (width 0.2) (layer "F.Cu") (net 1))
 (segment (start 139.39 61.19) (end 139.65 61.45) (width 0.2) (layer "F.Cu") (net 1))
 (segment (start 140.99 60.8191) (end 140.99 59.495) (width 0.2) (layer "F.Cu") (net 1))
 (via (at 156.21 61.9226) (size 0.6) (drill 0.3) (layers "F.Cu" "B.Cu") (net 1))
 (via (at 141.473 60.4856) (size 0.6) (drill 0.3) (layers "F.Cu" "B.Cu") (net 1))
 (segment (start 141.253 61.9226) (end 140.848 61.5182) (width 0.2) (layer "B.Cu") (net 1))
 (segment (start 140.848 61.5182) (end 140.848 61.11) (width 0.2) (layer "B.Cu") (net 1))
 (segment (start 140.848 61.11) (end 141.473 60.4856) (width 0.2) (layer "B.Cu") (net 1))
 (segment (start 156.21 61.9226) (end 141.253 61.9226) (width 0.2) (layer "B.Cu") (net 1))
 (segment (start 142.769 61.2848) (end 142.769 62.6062) (width 0.2) (layer "F.Cu") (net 26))
 (segment (start 142.769 62.6062) (end 141.875 63.5) (width 0.2) (layer "F.Cu") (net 26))
 (segment (start 153.936 59.4242) (end 153.936 61.3197) (width 0.2) (layer "F.Cu") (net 26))
 (segment (start 154.94 58.42) (end 153.936 59.4242) (width 0.2) (layer "F.Cu") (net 26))
 (via (at 153.936 61.3197) (size 0.6) (drill 0.3) (layers "F.Cu" "B.Cu") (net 26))
 (via (at 142.769 61.2848) (size 0.6) (drill 0.3) (layers "F.Cu" "B.Cu") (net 26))
 (segment (start 142.503 61.2848) (end 142.769 61.2848) (width 0.2) (layer "B.Cu") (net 26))
 (segment (start 142.468 61.3197) (end 141.25 61.3197) (width 0.2) (layer "B.Cu") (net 26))
 (segment (start 142.468 61.3197) (end 142.503 61.2848) (width 0.2) (layer "B.Cu") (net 26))
 (segment (start 153.936 61.3197) (end 142.468 61.3197) (width 0.2) (layer "B.Cu") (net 26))
 (segment (start 153.141 57.6794) (end 153.141 60.5508) (width 0.2) (layer "F.Cu") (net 2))
 (segment (start 144.087 60.5508) (end 144.087 61.0649) (width 0.2) (layer "F.Cu") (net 2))
 (segment (start 141.615 58.5929) (end 141.615 57.445) (width 0.2) (layer "F.Cu") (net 2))
 (segment (start 154.94 55.88) (end 153.141 57.6794) (width 0.2) (layer "F.Cu") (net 2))
 (segment (start 144.087 61.0649) (end 141.615 58.5929) (width 0.2) (layer "F.Cu") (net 2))
 (via (at 144.087 60.5508) (size 0.6) (drill 0.3) (layers "F.Cu" "B.Cu") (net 2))
 (via (at 153.141 60.5508) (size 0.6) (drill 0.3) (layers "F.Cu" "B.Cu") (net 2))
 (segment (start 144.087 60.5508) (end 153.141 60.5508) (width 0.2) (layer "B.Cu") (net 2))
 (segment (start 161.211 60.2621) (end 161.211 60.72) (width 0.2) (layer "F.Cu") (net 18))
 (segment (start 160.47 59.5211) (end 161.211 60.2621) (width 0.2) (layer "F.Cu") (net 18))
 (segment (start 144.78 58.172) (end 144.78 73.66) (width 0.2) (layer "F.Cu") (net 18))
 (via (at 160.47 59.5211) (size 0.6) (drill 0.3) (layers "F.Cu" "B.Cu") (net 18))
 (via (at 144.78 58.172) (size 0.6) (drill 0.3) (layers "F.Cu" "B.Cu") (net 18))
 (segment (start 155.4611 58.172) (end 156.8102 59.5211) (width 0.2) (layer "B.Cu") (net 18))
 (segment (start 144.78 58.172) (end 155.4611 58.172) (width 0.2) (layer "B.Cu") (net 18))
 (segment (start 160.47 59.5211) (end 156.8102 59.5211) (width 0.2) (layer "B.Cu") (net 18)))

